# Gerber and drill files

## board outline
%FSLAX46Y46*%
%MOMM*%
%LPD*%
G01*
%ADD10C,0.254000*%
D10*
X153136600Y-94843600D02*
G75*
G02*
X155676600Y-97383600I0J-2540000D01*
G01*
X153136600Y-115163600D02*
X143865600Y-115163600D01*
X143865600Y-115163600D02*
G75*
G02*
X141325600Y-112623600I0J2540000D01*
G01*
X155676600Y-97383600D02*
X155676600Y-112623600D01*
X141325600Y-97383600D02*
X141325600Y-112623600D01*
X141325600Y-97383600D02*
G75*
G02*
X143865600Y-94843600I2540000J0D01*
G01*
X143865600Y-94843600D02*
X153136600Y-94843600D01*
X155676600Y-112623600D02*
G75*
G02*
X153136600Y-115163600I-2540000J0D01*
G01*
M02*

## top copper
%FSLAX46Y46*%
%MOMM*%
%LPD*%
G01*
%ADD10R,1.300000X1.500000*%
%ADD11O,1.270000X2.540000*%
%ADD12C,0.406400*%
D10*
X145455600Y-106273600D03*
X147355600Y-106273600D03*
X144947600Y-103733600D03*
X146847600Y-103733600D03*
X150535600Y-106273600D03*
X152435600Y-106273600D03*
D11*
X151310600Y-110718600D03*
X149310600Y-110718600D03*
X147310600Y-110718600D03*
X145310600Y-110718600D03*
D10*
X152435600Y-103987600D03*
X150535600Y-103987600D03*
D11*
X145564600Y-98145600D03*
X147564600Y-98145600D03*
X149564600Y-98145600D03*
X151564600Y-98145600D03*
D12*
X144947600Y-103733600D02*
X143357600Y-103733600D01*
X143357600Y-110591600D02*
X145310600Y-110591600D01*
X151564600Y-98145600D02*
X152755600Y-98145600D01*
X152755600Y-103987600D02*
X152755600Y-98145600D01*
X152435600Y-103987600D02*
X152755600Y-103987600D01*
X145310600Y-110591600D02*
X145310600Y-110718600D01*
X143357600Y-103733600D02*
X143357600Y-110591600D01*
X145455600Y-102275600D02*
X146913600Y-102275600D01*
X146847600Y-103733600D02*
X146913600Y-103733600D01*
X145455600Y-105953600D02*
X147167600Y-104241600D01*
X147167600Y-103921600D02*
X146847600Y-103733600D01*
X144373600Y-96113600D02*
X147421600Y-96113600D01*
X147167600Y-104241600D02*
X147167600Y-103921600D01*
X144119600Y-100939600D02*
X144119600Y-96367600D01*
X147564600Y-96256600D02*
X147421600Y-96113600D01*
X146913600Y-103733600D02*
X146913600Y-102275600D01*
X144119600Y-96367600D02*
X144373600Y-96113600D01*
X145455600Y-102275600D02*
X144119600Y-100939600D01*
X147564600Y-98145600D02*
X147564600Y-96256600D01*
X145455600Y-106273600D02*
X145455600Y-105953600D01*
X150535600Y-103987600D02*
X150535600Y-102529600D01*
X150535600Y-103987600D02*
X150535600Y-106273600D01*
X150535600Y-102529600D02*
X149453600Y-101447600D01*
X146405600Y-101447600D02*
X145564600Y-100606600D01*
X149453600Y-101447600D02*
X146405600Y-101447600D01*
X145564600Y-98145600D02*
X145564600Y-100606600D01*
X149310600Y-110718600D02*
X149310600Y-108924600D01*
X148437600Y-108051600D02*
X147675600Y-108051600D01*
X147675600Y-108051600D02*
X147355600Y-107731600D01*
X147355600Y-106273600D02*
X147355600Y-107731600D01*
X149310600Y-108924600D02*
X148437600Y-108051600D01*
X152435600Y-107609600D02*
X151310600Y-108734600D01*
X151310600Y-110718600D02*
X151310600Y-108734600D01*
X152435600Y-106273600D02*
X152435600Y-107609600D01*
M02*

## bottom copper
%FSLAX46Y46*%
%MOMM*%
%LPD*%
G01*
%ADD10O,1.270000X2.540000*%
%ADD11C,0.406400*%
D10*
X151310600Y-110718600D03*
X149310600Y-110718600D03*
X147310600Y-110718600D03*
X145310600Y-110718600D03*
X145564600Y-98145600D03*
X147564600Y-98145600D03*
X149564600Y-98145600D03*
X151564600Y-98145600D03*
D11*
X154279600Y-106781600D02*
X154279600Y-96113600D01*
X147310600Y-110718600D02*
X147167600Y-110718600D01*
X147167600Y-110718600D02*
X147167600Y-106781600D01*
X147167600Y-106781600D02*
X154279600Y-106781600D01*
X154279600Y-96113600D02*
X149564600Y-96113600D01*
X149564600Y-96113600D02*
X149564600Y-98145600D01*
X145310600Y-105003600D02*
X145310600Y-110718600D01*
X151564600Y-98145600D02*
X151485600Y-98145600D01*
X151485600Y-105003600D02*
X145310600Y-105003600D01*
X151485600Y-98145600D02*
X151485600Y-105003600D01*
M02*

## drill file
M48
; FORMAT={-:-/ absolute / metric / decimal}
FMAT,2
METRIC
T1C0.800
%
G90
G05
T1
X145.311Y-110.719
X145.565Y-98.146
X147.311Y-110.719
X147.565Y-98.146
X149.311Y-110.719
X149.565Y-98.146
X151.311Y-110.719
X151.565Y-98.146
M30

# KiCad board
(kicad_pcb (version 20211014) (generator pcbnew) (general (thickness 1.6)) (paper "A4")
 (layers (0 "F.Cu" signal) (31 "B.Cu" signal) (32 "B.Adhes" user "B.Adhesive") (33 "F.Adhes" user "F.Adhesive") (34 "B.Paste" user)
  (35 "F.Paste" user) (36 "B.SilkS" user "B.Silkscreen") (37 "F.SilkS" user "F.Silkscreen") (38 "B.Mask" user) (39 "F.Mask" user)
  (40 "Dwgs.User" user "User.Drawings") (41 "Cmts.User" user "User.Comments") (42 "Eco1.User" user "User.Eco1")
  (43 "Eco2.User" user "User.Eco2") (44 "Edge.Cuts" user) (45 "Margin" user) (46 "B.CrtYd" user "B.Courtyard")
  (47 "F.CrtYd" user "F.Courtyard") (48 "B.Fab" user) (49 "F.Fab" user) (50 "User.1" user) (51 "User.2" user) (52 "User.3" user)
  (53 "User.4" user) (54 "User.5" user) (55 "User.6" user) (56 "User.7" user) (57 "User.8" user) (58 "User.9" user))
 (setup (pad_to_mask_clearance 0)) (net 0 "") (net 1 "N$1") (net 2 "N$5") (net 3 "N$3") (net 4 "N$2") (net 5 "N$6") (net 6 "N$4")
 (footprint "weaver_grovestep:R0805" (layer "F.Cu") (at 146.4056 106.2736)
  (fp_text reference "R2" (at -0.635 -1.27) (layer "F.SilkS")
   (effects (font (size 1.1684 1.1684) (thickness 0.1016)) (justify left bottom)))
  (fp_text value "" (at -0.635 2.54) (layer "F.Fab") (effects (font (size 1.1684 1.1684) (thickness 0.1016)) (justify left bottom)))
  (pad "1" smd rect (at -0.95 0) (size 1.3 1.5) (layers "F.Cu" "F.Paste" "F.Mask") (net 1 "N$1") (solder_mask_margin 0.1016))
  (pad "2" smd rect (at 0.95 0) (size 1.3 1.5) (layers "F.Cu" "F.Paste" "F.Mask") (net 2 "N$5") (solder_mask_margin 0.1016)))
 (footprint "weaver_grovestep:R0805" (layer "F.Cu") (at 145.8976 103.7336)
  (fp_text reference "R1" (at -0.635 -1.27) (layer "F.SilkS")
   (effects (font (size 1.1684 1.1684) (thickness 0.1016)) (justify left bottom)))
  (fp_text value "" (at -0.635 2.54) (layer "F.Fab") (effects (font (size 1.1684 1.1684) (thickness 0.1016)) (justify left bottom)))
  (pad "1" smd rect (at -0.95 0) (size 1.3 1.5) (layers "F.Cu" "F.Paste" "F.Mask") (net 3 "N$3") (solder_mask_margin 0.1016))
  (pad "2" smd rect (at 0.95 0) (size 1.3 1.5) (layers "F.Cu" "F.Paste" "F.Mask") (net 1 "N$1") (solder_mask_margin 0.1016)))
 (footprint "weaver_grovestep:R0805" (layer "F.Cu") (at 151.4856 106.2736)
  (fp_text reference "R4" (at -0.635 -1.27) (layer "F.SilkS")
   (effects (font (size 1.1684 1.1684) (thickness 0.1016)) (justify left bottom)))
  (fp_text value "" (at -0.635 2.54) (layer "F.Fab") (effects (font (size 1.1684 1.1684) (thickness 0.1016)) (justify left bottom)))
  (pad "1" smd rect (at -0.95 0) (size 1.3 1.5) (layers "F.Cu" "F.Paste" "F.Mask") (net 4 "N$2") (solder_mask_margin 0.1016))
  (pad "2" smd rect (at 0.95 0) (size 1.3 1.5) (layers "F.Cu" "F.Paste" "F.Mask") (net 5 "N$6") (solder_mask_margin 0.1016)))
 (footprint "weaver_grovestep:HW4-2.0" (layer "F.Cu") (at 148.3106 110.7186 180)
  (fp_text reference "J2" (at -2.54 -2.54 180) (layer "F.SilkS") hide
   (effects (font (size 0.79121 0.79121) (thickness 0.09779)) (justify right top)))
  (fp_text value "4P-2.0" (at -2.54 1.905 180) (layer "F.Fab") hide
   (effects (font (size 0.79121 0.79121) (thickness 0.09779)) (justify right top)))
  (pad "1" thru_hole oval (at -3 0 270) (size 2.54 1.27) (drill 0.8) (layers *.Cu *.Mask) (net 5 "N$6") (solder_mask_margin 0.1016))
  (pad "2" thru_hole oval (at -1 0 270) (size 2.54 1.27) (drill 0.8) (layers *.Cu *.Mask) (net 2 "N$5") (solder_mask_margin 0.1016))
  (pad "3" thru_hole oval (at 1 0 270) (size 2.54 1.27) (drill 0.8) (layers *.Cu *.Mask) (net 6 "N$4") (solder_mask_margin 0.1016))
  (pad "4" thru_hole oval (at 3 0 270) (size 2.54 1.27) (drill 0.8) (layers *.Cu *.Mask) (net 3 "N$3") (solder_mask_margin 0.1016)))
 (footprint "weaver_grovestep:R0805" (layer "F.Cu") (at 151.4856 103.9876 180)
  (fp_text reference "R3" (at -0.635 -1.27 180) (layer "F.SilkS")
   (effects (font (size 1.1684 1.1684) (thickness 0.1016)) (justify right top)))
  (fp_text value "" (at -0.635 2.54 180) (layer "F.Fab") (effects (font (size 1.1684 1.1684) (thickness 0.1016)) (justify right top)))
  (pad "1" smd rect (at -0.95 0 180) (size 1.3 1.5) (layers "F.Cu" "F.Paste" "F.Mask") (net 3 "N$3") (solder_mask_margin 0.1016))
  (pad "2" smd rect (at 0.95 0 180) (size 1.3 1.5) (layers "F.Cu" "F.Paste" "F.Mask") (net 4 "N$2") (solder_mask_margin 0.1016)))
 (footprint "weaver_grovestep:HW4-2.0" (layer "F.Cu") (at 148.5646 98.1456)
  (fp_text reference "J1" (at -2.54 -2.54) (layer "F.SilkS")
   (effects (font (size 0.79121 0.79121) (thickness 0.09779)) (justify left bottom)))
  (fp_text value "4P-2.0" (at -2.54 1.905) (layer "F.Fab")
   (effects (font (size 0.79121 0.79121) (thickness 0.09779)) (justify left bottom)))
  (pad "1" thru_hole oval (at -3 0 90) (size 2.54 1.27) (drill 0.8) (layers *.Cu *.Mask) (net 4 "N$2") (solder_mask_margin 0.1016))
  (pad "2" thru_hole oval (at -1 0 90) (size 2.54 1.27) (drill 0.8) (layers *.Cu *.Mask) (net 1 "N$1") (solder_mask_margin 0.1016))
  (pad "3" thru_hole oval (at 1 0 90) (size 2.54 1.27) (drill 0.8) (layers *.Cu *.Mask) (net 6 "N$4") (solder_mask_margin 0.1016))
  (pad "4" thru_hole oval (at 3 0 90) (size 2.54 1.27) (drill 0.8) (layers *.Cu *.Mask) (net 3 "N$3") (solder_mask_margin 0.1016)))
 (gr_arc (start 153.1366 94.8436) (mid 154.932651 95.587549) (end 155.6766 97.3836) (layer "Edge.Cuts") (width 0.254))
 (gr_line (start 153.1366 115.1636) (end 143.8656 115.1636) (layer "Edge.Cuts") (width 0.254))
 (gr_arc (start 143.8656 115.1636) (mid 142.069549 114.419651) (end 141.3256 112.6236) (layer "Edge.Cuts") (width 0.254))
 (gr_line (start 155.6766 97.3836) (end 155.6766 112.6236) (layer "Edge.Cuts") (width 0.254))
 (gr_line (start 141.3256 97.3836) (end 141.3256 112.6236) (layer "Edge.Cuts") (width 0.254))
 (gr_arc (start 141.3256 97.3836) (mid 142.069549 95.587549) (end 143.8656 94.8436) (layer "Edge.Cuts") (width 0.254))
 (gr_line (start 143.8656 94.8436) (end 153.1366 94.8436) (layer "Edge.Cuts") (width 0.254))
 (gr_arc (start 155.6766 112.6236) (mid 154.932651 114.419651) (end 153.1366 115.1636) (layer "Edge.Cuts") (width 0.254))
 (segment (start 154.2796 106.7816) (end 154.2796 96.1136) (width 0.4064) (layer "B.Cu") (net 6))
 (segment (start 147.3106 110.7186) (end 147.1676 110.7186) (width 0.4064) (layer "B.Cu") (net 6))
 (segment (start 147.1676 110.7186) (end 147.1676 106.7816) (width 0.4064) (layer "B.Cu") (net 6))
 (segment (start 147.1676 106.7816) (end 154.2796 106.7816) (width 0.4064) (layer "B.Cu") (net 6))
 (segment (start 154.2796 96.1136) (end 149.5646 96.1136) (width 0.4064) (layer "B.Cu") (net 6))
 (segment (start 149.5646 96.1136) (end 149.5646 98.1456) (width 0.4064) (layer "B.Cu") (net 6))
 (segment (start 144.9476 103.7336) (end 143.3576 103.7336) (width 0.4064) (layer "F.Cu") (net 3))
 (segment (start 143.3576 110.5916) (end 145.3106 110.5916) (width 0.4064) (layer "F.Cu") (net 3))
 (segment (start 151.5646 98.1456) (end 152.7556 98.1456) (width 0.4064) (layer "F.Cu") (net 3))
 (segment (start 152.7556 103.9876) (end 152.7556 98.1456) (width 0.4064) (layer "F.Cu") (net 3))
 (segment (start 152.4356 103.9876) (end 152.7556 103.9876) (width 0.4064) (layer "F.Cu") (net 3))
 (segment (start 145.3106 110.5916) (end 145.3106 110.7186) (width 0.4064) (layer "F.Cu") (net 3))
 (segment (start 143.3576 103.7336) (end 143.3576 110.5916) (width 0.4064) (layer "F.Cu") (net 3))
 (segment (start 145.3106 105.0036) (end 145.3106 110.7186) (width 0.4064) (layer "B.Cu") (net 3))
 (segment (start 151.5646 98.1456) (end 151.4856 98.1456) (width 0.4064) (layer "B.Cu") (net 3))
 (segment (start 151.4856 105.0036) (end 145.3106 105.0036) (width 0.4064) (layer "B.Cu") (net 3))
 (segment (start 151.4856 98.1456) (end 151.4856 105.0036) (width 0.4064) (layer "B.Cu") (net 3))
 (segment (start 145.4556 102.2756) (end 146.9136 102.2756) (width 0.4064) (layer "F.Cu") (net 1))
 (segment (start 146.8476 103.7336) (end 146.9136 103.7336) (width 0.4064) (layer "F.Cu") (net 1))
 (segment (start 145.4556 105.9536) (end 147.1676 104.2416) (width 0.4064) (layer "F.Cu") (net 1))
 (segment (start 147.1676 103.9216) (end 146.8476 103.7336) (width 0.4064) (layer "F.Cu") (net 1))
 (segment (start 144.3736 96.1136) (end 147.4216 96.1136) (width 0.4064) (layer "F.Cu") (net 1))
 (segment (start 147.1676 104.2416) (end 147.1676 103.9216) (width 0.4064) (layer "F.Cu") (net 1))
 (segment (start 144.1196 100.9396) (end 144.1196 96.3676) (width 0.4064) (layer "F.Cu") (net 1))
 (segment (start 147.5646 96.2566) (end 147.4216 96.1136) (width 0.4064) (layer "F.Cu") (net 1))
 (segment (start 146.9136 103.7336) (end 146.9136 102.2756) (width 0.4064) (layer "F.Cu") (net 1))
 (segment (start 144.1196 96.3676) (end 144.3736 96.1136) (width 0.4064) (layer "F.Cu") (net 1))
 (segment (start 145.4556 102.2756) (end 144.1196 100.9396) (width 0.4064) (layer "F.Cu") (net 1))
 (segment (start 147.5646 98.1456) (end 147.5646 96.2566) (width 0.4064) (layer "F.Cu") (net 1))
 (segment (start 145.4556 106.2736) (end 145.4556 105.9536) (width 0.4064) (layer "F.Cu") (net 1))
 (segment (start 150.5356 103.9876) (end 150.5356 102.5296) (width 0.4064) (layer "F.Cu") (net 4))
 (segment (start 150.5356 103.9876) (end 150.5356 106.2736) (width 0.4064) (layer "F.Cu") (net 4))
 (segment (start 150.5356 102.5296) (end 149.4536 101.4476) (width 0.4064) (layer "F.Cu") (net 4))
 (segment (start 146.4056 101.4476) (end 145.5646 100.6066) (width 0.4064) (layer "F.Cu") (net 4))
 (segment (start 149.4536 101.4476) (end 146.4056 101.4476) (width 0.4064) (layer "F.Cu") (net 4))
 (segment (start 145.5646 98.1456) (end 145.5646 100.6066) (width 0.4064) (layer "F.Cu") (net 4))
 (segment (start 149.3106 110.7186) (end 149.3106 108.9246) (width 0.4064) (layer "F.Cu") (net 2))
 (segment (start 148.4376 108.0516) (end 147.6756 108.0516) (width 0.4064) (layer "F.Cu") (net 2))
 (segment (start 147.6756 108.0516) (end 147.3556 107.7316) (width 0.4064) (layer "F.Cu") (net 2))
 (segment (start 147.3556 106.2736) (end 147.3556 107.7316) (width 0.4064) (layer "F.Cu") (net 2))
 (segment (start 149.3106 108.9246) (end 148.4376 108.0516) (width 0.4064) (layer "F.Cu") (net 2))
 (segment (start 152.4356 107.6096) (end 151.3106 108.7346) (width 0.4064) (layer "F.Cu") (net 5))
 (segment (start 151.3106 110.7186) (end 151.3106 108.7346) (width 0.4064) (layer "F.Cu") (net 5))
 (segment (start 152.4356 106.2736) (end 152.4356 107.6096) (width 0.4064) (layer "F.Cu") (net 5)))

